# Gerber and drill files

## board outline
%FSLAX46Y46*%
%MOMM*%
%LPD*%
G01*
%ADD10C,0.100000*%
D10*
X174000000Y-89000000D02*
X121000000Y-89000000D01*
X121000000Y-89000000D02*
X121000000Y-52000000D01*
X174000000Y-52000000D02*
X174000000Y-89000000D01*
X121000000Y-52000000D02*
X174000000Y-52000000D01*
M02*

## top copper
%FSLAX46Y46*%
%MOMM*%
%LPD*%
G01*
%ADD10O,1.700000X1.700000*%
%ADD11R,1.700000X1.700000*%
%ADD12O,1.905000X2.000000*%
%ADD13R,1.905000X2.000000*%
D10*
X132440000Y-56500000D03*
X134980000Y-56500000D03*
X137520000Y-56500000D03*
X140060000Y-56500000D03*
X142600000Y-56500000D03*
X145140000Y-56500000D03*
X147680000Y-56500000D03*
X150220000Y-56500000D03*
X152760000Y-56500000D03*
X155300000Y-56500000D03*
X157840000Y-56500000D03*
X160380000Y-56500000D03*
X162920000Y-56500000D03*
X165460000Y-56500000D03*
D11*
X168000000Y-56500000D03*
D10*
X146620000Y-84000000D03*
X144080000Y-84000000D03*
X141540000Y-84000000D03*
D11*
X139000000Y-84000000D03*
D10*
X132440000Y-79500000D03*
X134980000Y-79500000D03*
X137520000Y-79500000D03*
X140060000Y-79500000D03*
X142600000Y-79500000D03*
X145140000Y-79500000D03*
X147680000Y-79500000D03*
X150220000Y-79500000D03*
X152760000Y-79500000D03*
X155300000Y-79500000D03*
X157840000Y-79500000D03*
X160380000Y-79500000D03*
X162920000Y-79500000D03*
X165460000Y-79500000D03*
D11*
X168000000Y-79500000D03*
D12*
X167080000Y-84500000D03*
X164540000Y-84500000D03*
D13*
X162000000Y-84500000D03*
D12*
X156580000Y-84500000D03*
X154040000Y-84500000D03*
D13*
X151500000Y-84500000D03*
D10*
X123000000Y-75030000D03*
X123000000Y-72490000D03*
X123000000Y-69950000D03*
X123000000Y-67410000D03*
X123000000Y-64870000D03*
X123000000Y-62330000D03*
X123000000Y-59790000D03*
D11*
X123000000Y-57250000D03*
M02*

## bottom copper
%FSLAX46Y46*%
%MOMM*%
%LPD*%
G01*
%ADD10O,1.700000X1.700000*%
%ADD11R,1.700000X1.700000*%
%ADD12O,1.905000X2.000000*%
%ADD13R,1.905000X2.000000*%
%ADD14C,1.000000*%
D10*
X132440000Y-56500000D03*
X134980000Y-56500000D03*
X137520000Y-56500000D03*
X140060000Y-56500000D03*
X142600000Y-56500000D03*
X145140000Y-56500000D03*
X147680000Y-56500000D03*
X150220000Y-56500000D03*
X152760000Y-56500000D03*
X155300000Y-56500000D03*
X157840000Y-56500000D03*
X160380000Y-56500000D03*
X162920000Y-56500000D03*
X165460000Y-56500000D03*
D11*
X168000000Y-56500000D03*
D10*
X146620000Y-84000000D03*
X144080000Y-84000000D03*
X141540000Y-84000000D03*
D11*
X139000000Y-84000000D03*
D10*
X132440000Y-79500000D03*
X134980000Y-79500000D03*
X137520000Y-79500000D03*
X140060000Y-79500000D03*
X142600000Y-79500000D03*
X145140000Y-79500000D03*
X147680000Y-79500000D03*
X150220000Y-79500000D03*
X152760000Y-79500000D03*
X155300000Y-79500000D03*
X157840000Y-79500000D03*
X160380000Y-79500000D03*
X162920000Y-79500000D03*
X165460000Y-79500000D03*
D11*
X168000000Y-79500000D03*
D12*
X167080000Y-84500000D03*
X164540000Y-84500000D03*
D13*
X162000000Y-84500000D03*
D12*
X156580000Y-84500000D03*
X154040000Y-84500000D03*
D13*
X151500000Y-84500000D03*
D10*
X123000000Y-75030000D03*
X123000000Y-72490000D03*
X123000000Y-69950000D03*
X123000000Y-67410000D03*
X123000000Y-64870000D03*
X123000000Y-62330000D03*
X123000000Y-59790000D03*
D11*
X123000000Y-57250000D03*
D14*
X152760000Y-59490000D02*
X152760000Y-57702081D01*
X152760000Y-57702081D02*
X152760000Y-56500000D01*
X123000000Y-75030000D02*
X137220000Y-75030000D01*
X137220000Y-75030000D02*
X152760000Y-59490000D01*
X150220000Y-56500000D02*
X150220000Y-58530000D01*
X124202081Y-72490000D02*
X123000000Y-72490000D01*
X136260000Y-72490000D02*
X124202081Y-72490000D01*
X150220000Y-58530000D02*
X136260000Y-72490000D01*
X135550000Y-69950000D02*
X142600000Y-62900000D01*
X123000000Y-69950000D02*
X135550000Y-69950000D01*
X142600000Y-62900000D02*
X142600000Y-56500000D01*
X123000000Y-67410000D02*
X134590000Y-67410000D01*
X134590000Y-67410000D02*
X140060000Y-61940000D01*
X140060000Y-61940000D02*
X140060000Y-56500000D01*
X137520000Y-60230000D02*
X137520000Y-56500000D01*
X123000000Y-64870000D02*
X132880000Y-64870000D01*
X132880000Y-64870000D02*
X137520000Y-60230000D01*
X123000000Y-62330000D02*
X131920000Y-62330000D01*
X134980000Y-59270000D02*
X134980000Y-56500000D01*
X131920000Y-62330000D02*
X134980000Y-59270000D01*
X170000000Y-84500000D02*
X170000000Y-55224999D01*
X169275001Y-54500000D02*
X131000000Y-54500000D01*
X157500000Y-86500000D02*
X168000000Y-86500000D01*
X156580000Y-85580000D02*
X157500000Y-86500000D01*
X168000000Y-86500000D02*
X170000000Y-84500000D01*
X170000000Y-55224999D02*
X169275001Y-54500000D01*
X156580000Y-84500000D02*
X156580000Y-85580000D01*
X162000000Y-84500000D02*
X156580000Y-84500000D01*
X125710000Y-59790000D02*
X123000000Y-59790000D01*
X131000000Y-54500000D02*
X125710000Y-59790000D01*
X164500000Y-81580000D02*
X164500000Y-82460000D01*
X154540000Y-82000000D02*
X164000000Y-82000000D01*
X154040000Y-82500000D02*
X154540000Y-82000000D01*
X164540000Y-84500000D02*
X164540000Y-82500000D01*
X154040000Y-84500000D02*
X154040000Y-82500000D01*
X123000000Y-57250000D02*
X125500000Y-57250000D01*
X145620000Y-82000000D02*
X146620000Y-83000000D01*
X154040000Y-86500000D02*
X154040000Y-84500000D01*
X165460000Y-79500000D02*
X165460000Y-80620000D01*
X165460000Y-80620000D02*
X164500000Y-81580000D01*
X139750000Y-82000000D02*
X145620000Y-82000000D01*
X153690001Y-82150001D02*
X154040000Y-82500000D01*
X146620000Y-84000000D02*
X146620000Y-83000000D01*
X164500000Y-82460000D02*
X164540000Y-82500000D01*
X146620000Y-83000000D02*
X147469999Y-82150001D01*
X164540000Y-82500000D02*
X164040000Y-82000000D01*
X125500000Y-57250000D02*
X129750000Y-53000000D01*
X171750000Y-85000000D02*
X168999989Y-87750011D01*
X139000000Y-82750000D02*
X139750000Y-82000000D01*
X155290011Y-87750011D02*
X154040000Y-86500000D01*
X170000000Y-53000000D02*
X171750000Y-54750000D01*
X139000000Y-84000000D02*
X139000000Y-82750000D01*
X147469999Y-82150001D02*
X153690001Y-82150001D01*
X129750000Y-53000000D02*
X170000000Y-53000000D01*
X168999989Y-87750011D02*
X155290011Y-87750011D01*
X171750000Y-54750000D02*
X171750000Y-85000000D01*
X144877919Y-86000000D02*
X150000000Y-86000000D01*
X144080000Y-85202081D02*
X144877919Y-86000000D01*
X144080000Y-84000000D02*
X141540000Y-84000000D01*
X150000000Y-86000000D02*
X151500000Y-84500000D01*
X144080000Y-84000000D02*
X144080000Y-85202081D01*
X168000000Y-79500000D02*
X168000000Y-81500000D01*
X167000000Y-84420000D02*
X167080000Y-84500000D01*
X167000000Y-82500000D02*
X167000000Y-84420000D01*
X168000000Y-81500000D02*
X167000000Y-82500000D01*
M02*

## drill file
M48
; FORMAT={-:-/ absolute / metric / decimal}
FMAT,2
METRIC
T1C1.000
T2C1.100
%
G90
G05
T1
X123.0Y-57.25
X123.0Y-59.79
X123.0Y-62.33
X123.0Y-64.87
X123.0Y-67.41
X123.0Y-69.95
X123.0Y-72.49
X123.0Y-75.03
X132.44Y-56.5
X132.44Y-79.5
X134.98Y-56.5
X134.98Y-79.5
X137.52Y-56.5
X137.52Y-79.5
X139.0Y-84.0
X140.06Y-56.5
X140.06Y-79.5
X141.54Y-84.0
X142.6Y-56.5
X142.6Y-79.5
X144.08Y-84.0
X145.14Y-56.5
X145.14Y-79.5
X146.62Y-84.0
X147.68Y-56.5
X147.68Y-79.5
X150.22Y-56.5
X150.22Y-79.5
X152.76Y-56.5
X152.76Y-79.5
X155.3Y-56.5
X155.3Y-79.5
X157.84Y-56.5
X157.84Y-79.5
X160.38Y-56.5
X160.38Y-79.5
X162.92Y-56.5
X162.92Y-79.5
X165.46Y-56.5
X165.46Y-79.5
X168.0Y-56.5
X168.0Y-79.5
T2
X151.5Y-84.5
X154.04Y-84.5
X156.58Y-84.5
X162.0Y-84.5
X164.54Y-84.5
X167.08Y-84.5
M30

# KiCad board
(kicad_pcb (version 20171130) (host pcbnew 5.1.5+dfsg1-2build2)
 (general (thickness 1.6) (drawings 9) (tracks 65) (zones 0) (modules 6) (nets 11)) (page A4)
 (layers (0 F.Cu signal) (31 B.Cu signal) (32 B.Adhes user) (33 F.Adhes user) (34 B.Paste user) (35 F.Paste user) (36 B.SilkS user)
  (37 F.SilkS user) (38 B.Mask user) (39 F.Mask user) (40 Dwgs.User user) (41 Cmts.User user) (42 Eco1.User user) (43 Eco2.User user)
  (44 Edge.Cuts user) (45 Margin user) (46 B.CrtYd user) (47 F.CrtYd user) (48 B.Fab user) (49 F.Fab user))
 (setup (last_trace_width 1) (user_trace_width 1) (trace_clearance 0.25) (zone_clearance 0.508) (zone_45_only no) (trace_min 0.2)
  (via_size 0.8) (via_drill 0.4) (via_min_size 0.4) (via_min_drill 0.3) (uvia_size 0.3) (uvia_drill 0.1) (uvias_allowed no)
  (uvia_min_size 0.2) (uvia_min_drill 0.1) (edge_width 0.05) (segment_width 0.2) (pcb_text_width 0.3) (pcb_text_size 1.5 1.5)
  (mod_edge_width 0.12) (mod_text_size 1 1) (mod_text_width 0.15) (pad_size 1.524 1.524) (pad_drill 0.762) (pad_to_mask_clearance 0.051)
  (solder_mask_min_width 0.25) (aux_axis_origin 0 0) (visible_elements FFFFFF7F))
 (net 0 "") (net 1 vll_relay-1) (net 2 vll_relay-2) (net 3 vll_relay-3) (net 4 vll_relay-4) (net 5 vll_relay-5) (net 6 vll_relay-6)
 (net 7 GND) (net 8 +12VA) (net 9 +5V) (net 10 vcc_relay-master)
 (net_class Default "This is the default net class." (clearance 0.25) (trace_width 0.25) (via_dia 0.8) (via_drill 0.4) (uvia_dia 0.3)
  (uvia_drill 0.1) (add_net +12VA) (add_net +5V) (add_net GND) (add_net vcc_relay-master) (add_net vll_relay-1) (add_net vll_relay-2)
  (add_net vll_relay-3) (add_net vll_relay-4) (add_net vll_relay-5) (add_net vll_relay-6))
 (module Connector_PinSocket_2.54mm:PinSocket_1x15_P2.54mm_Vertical (layer F.Cu) (at 168 56.5 270)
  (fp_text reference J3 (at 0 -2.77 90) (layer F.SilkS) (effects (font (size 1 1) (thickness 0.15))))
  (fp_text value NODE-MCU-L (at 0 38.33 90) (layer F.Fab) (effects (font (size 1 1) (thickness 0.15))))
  (pad 15 thru_hole oval (at 0 35.56 270) (size 1.7 1.7) (drill 1) (layers *.Cu *.Mask))
  (pad 14 thru_hole oval (at 0 33.02 270) (size 1.7 1.7) (drill 1) (layers *.Cu *.Mask) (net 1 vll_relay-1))
  (pad 13 thru_hole oval (at 0 30.48 270) (size 1.7 1.7) (drill 1) (layers *.Cu *.Mask) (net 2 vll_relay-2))
  (pad 12 thru_hole oval (at 0 27.94 270) (size 1.7 1.7) (drill 1) (layers *.Cu *.Mask) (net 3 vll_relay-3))
  (pad 11 thru_hole oval (at 0 25.4 270) (size 1.7 1.7) (drill 1) (layers *.Cu *.Mask) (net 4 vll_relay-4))
  (pad 10 thru_hole oval (at 0 22.86 270) (size 1.7 1.7) (drill 1) (layers *.Cu *.Mask))
  (pad 9 thru_hole oval (at 0 20.32 270) (size 1.7 1.7) (drill 1) (layers *.Cu *.Mask))
  (pad 8 thru_hole oval (at 0 17.78 270) (size 1.7 1.7) (drill 1) (layers *.Cu *.Mask) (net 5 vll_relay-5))
  (pad 7 thru_hole oval (at 0 15.24 270) (size 1.7 1.7) (drill 1) (layers *.Cu *.Mask) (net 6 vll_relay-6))
  (pad 6 thru_hole oval (at 0 12.7 270) (size 1.7 1.7) (drill 1) (layers *.Cu *.Mask))
  (pad 5 thru_hole oval (at 0 10.16 270) (size 1.7 1.7) (drill 1) (layers *.Cu *.Mask))
  (pad 4 thru_hole oval (at 0 7.62 270) (size 1.7 1.7) (drill 1) (layers *.Cu *.Mask))
  (pad 3 thru_hole oval (at 0 5.08 270) (size 1.7 1.7) (drill 1) (layers *.Cu *.Mask))
  (pad 2 thru_hole oval (at 0 2.54 270) (size 1.7 1.7) (drill 1) (layers *.Cu *.Mask))
  (pad 1 thru_hole rect (at 0 0 270) (size 1.7 1.7) (drill 1) (layers *.Cu *.Mask)))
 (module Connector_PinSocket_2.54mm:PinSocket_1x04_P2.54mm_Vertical (layer F.Cu) (at 139 84 90)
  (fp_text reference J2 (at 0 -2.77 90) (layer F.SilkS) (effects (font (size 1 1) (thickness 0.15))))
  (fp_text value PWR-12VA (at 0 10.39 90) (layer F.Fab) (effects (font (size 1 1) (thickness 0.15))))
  (pad 4 thru_hole oval (at 0 7.62 90) (size 1.7 1.7) (drill 1) (layers *.Cu *.Mask) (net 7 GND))
  (pad 3 thru_hole oval (at 0 5.08 90) (size 1.7 1.7) (drill 1) (layers *.Cu *.Mask) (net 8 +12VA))
  (pad 2 thru_hole oval (at 0 2.54 90) (size 1.7 1.7) (drill 1) (layers *.Cu *.Mask) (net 8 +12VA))
  (pad 1 thru_hole rect (at 0 0 90) (size 1.7 1.7) (drill 1) (layers *.Cu *.Mask) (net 7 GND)))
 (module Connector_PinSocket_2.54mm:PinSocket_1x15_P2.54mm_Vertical (layer F.Cu) (at 168 79.5 270)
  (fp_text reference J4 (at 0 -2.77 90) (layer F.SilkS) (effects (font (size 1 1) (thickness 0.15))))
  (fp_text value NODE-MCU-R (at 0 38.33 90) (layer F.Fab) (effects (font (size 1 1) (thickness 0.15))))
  (pad 15 thru_hole oval (at 0 35.56 270) (size 1.7 1.7) (drill 1) (layers *.Cu *.Mask))
  (pad 14 thru_hole oval (at 0 33.02 270) (size 1.7 1.7) (drill 1) (layers *.Cu *.Mask))
  (pad 13 thru_hole oval (at 0 30.48 270) (size 1.7 1.7) (drill 1) (layers *.Cu *.Mask))
  (pad 12 thru_hole oval (at 0 27.94 270) (size 1.7 1.7) (drill 1) (layers *.Cu *.Mask))
  (pad 11 thru_hole oval (at 0 25.4 270) (size 1.7 1.7) (drill 1) (layers *.Cu *.Mask))
  (pad 10 thru_hole oval (at 0 22.86 270) (size 1.7 1.7) (drill 1) (layers *.Cu *.Mask))
  (pad 9 thru_hole oval (at 0 20.32 270) (size 1.7 1.7) (drill 1) (layers *.Cu *.Mask))
  (pad 8 thru_hole oval (at 0 17.78 270) (size 1.7 1.7) (drill 1) (layers *.Cu *.Mask))
  (pad 7 thru_hole oval (at 0 15.24 270) (size 1.7 1.7) (drill 1) (layers *.Cu *.Mask))
  (pad 6 thru_hole oval (at 0 12.7 270) (size 1.7 1.7) (drill 1) (layers *.Cu *.Mask))
  (pad 5 thru_hole oval (at 0 10.16 270) (size 1.7 1.7) (drill 1) (layers *.Cu *.Mask))
  (pad 4 thru_hole oval (at 0 7.62 270) (size 1.7 1.7) (drill 1) (layers *.Cu *.Mask))
  (pad 3 thru_hole oval (at 0 5.08 270) (size 1.7 1.7) (drill 1) (layers *.Cu *.Mask))
  (pad 2 thru_hole oval (at 0 2.54 270) (size 1.7 1.7) (drill 1) (layers *.Cu *.Mask) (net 7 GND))
  (pad 1 thru_hole rect (at 0 0 270) (size 1.7 1.7) (drill 1) (layers *.Cu *.Mask) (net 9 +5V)))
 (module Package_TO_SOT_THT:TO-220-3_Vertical (layer F.Cu) (at 162 84.5)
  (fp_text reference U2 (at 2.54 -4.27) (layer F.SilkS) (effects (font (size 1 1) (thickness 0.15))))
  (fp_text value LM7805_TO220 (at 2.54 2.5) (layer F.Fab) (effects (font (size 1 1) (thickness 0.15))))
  (pad 3 thru_hole oval (at 5.08 0) (size 1.905 2) (drill 1.1) (layers *.Cu *.Mask) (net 9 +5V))
  (pad 2 thru_hole oval (at 2.54 0) (size 1.905 2) (drill 1.1) (layers *.Cu *.Mask) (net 7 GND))
  (pad 1 thru_hole rect (at 0 0) (size 1.905 2) (drill 1.1) (layers *.Cu *.Mask) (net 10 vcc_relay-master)))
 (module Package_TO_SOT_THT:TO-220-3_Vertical (layer F.Cu) (at 151.5 84.5)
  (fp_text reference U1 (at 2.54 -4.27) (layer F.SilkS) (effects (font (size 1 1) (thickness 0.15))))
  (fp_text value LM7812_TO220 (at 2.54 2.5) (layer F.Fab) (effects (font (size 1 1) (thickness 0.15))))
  (pad 3 thru_hole oval (at 5.08 0) (size 1.905 2) (drill 1.1) (layers *.Cu *.Mask) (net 10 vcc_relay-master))
  (pad 2 thru_hole oval (at 2.54 0) (size 1.905 2) (drill 1.1) (layers *.Cu *.Mask) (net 7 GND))
  (pad 1 thru_hole rect (at 0 0) (size 1.905 2) (drill 1.1) (layers *.Cu *.Mask) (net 8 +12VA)))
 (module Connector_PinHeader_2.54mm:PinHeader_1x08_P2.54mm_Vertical (layer F.Cu) (at 123 57.25)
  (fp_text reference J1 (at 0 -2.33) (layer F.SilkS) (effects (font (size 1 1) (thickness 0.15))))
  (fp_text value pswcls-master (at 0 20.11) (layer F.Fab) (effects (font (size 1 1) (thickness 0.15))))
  (pad 8 thru_hole oval (at 0 17.78) (size 1.7 1.7) (drill 1) (layers *.Cu *.Mask) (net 6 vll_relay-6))
  (pad 7 thru_hole oval (at 0 15.24) (size 1.7 1.7) (drill 1) (layers *.Cu *.Mask) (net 5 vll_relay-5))
  (pad 6 thru_hole oval (at 0 12.7) (size 1.7 1.7) (drill 1) (layers *.Cu *.Mask) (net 4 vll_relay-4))
  (pad 5 thru_hole oval (at 0 10.16) (size 1.7 1.7) (drill 1) (layers *.Cu *.Mask) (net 3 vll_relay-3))
  (pad 4 thru_hole oval (at 0 7.62) (size 1.7 1.7) (drill 1) (layers *.Cu *.Mask) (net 2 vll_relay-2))
  (pad 3 thru_hole oval (at 0 5.08) (size 1.7 1.7) (drill 1) (layers *.Cu *.Mask) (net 1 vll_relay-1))
  (pad 2 thru_hole oval (at 0 2.54) (size 1.7 1.7) (drill 1) (layers *.Cu *.Mask) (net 10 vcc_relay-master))
  (pad 1 thru_hole rect (at 0 0) (size 1.7 1.7) (drill 1) (layers *.Cu *.Mask) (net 7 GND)))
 (gr_line (start 174 89) (end 121 89) (layer Edge.Cuts) (width 0.1))
 (gr_line (start 121 89) (end 121 52) (layer Edge.Cuts) (width 0.1))
 (gr_line (start 174 52) (end 174 89) (layer Edge.Cuts) (width 0.1))
 (gr_line (start 121 52) (end 174 52) (layer Edge.Cuts) (width 0.1))
 (segment (start 152.76 59.49) (end 152.76 57.702081) (width 1) (layer B.Cu) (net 6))
 (segment (start 152.76 57.702081) (end 152.76 56.5) (width 1) (layer B.Cu) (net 6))
 (segment (start 123 75.03) (end 137.22 75.03) (width 1) (layer B.Cu) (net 6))
 (segment (start 137.22 75.03) (end 152.76 59.49) (width 1) (layer B.Cu) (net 6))
 (segment (start 150.22 56.5) (end 150.22 58.53) (width 1) (layer B.Cu) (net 5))
 (segment (start 124.202081 72.49) (end 123 72.49) (width 1) (layer B.Cu) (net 5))
 (segment (start 136.26 72.49) (end 124.202081 72.49) (width 1) (layer B.Cu) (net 5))
 (segment (start 150.22 58.53) (end 136.26 72.49) (width 1) (layer B.Cu) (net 5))
 (segment (start 135.55 69.95) (end 142.6 62.9) (width 1) (layer B.Cu) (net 4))
 (segment (start 123 69.95) (end 135.55 69.95) (width 1) (layer B.Cu) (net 4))
 (segment (start 142.6 62.9) (end 142.6 56.5) (width 1) (layer B.Cu) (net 4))
 (segment (start 123 67.41) (end 134.59 67.41) (width 1) (layer B.Cu) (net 3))
 (segment (start 134.59 67.41) (end 140.06 61.94) (width 1) (layer B.Cu) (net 3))
 (segment (start 140.06 61.94) (end 140.06 56.5) (width 1) (layer B.Cu) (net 3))
 (segment (start 137.52 60.23) (end 137.52 56.5) (width 1) (layer B.Cu) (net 2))
 (segment (start 123 64.87) (end 132.88 64.87) (width 1) (layer B.Cu) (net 2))
 (segment (start 132.88 64.87) (end 137.52 60.23) (width 1) (layer B.Cu) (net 2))
 (segment (start 123 62.33) (end 131.92 62.33) (width 1) (layer B.Cu) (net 1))
 (segment (start 134.98 59.27) (end 134.98 56.5) (width 1) (layer B.Cu) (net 1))
 (segment (start 131.92 62.33) (end 134.98 59.27) (width 1) (layer B.Cu) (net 1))
 (segment (start 170 84.5) (end 170 55.224999) (width 1) (layer B.Cu) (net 10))
 (segment (start 169.275001 54.5) (end 131 54.5) (width 1) (layer B.Cu) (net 10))
 (segment (start 157.5 86.5) (end 168 86.5) (width 1) (layer B.Cu) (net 10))
 (segment (start 156.58 85.58) (end 157.5 86.5) (width 1) (layer B.Cu) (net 10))
 (segment (start 168 86.5) (end 170 84.5) (width 1) (layer B.Cu) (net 10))
 (segment (start 170 55.224999) (end 169.275001 54.5) (width 1) (layer B.Cu) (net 10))
 (segment (start 156.58 84.5) (end 156.58 85.58) (width 1) (layer B.Cu) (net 10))
 (segment (start 162 84.5) (end 156.58 84.5) (width 1) (layer B.Cu) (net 10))
 (segment (start 125.71 59.79) (end 123 59.79) (width 1) (layer B.Cu) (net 10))
 (segment (start 131 54.5) (end 125.71 59.79) (width 1) (layer B.Cu) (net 10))
 (segment (start 164.5 81.58) (end 164.5 82.46) (width 1) (layer B.Cu) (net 7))
 (segment (start 154.54 82) (end 164 82) (width 1) (layer B.Cu) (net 7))
 (segment (start 154.04 82.5) (end 154.54 82) (width 1) (layer B.Cu) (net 7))
 (segment (start 164.54 84.5) (end 164.54 82.5) (width 1) (layer B.Cu) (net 7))
 (segment (start 154.04 84.5) (end 154.04 82.5) (width 1) (layer B.Cu) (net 7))
 (segment (start 123 57.25) (end 125.5 57.25) (width 1) (layer B.Cu) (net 7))
 (segment (start 145.62 82) (end 146.62 83) (width 1) (layer B.Cu) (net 7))
 (segment (start 154.04 86.5) (end 154.04 84.5) (width 1) (layer B.Cu) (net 7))
 (segment (start 165.46 79.5) (end 165.46 80.62) (width 1) (layer B.Cu) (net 7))
 (segment (start 165.46 80.62) (end 164.5 81.58) (width 1) (layer B.Cu) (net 7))
 (segment (start 139.75 82) (end 145.62 82) (width 1) (layer B.Cu) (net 7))
 (segment (start 153.690001 82.150001) (end 154.04 82.5) (width 1) (layer B.Cu) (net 7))
 (segment (start 146.62 84) (end 146.62 83) (width 1) (layer B.Cu) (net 7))
 (segment (start 164.5 82.46) (end 164.54 82.5) (width 1) (layer B.Cu) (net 7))
 (segment (start 146.62 83) (end 147.469999 82.150001) (width 1) (layer B.Cu) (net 7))
 (segment (start 164.54 82.5) (end 164.04 82) (width 1) (layer B.Cu) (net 7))
 (segment (start 125.5 57.25) (end 129.75 53) (width 1) (layer B.Cu) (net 7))
 (segment (start 171.75 85) (end 168.999989 87.750011) (width 1) (layer B.Cu) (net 7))
 (segment (start 139 82.75) (end 139.75 82) (width 1) (layer B.Cu) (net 7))
 (segment (start 155.290011 87.750011) (end 154.04 86.5) (width 1) (layer B.Cu) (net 7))
 (segment (start 170 53) (end 171.75 54.75) (width 1) (layer B.Cu) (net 7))
 (segment (start 139 84) (end 139 82.75) (width 1) (layer B.Cu) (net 7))
 (segment (start 147.469999 82.150001) (end 153.690001 82.150001) (width 1) (layer B.Cu) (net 7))
 (segment (start 129.75 53) (end 170 53) (width 1) (layer B.Cu) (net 7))
 (segment (start 168.999989 87.750011) (end 155.290011 87.750011) (width 1) (layer B.Cu) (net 7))
 (segment (start 171.75 54.75) (end 171.75 85) (width 1) (layer B.Cu) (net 7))
 (segment (start 144.877919 86) (end 150 86) (width 1) (layer B.Cu) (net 8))
 (segment (start 144.08 85.202081) (end 144.877919 86) (width 1) (layer B.Cu) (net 8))
 (segment (start 144.08 84) (end 141.54 84) (width 1) (layer B.Cu) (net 8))
 (segment (start 150 86) (end 151.5 84.5) (width 1) (layer B.Cu) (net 8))
 (segment (start 144.08 84) (end 144.08 85.202081) (width 1) (layer B.Cu) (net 8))
 (segment (start 168 79.5) (end 168 81.5) (width 1) (layer B.Cu) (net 9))
 (segment (start 167 84.42) (end 167.08 84.5) (width 1) (layer B.Cu) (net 9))
 (segment (start 167 82.5) (end 167 84.42) (width 1) (layer B.Cu) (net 9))
 (segment (start 168 81.5) (end 167 82.5) (width 1) (layer B.Cu) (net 9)))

